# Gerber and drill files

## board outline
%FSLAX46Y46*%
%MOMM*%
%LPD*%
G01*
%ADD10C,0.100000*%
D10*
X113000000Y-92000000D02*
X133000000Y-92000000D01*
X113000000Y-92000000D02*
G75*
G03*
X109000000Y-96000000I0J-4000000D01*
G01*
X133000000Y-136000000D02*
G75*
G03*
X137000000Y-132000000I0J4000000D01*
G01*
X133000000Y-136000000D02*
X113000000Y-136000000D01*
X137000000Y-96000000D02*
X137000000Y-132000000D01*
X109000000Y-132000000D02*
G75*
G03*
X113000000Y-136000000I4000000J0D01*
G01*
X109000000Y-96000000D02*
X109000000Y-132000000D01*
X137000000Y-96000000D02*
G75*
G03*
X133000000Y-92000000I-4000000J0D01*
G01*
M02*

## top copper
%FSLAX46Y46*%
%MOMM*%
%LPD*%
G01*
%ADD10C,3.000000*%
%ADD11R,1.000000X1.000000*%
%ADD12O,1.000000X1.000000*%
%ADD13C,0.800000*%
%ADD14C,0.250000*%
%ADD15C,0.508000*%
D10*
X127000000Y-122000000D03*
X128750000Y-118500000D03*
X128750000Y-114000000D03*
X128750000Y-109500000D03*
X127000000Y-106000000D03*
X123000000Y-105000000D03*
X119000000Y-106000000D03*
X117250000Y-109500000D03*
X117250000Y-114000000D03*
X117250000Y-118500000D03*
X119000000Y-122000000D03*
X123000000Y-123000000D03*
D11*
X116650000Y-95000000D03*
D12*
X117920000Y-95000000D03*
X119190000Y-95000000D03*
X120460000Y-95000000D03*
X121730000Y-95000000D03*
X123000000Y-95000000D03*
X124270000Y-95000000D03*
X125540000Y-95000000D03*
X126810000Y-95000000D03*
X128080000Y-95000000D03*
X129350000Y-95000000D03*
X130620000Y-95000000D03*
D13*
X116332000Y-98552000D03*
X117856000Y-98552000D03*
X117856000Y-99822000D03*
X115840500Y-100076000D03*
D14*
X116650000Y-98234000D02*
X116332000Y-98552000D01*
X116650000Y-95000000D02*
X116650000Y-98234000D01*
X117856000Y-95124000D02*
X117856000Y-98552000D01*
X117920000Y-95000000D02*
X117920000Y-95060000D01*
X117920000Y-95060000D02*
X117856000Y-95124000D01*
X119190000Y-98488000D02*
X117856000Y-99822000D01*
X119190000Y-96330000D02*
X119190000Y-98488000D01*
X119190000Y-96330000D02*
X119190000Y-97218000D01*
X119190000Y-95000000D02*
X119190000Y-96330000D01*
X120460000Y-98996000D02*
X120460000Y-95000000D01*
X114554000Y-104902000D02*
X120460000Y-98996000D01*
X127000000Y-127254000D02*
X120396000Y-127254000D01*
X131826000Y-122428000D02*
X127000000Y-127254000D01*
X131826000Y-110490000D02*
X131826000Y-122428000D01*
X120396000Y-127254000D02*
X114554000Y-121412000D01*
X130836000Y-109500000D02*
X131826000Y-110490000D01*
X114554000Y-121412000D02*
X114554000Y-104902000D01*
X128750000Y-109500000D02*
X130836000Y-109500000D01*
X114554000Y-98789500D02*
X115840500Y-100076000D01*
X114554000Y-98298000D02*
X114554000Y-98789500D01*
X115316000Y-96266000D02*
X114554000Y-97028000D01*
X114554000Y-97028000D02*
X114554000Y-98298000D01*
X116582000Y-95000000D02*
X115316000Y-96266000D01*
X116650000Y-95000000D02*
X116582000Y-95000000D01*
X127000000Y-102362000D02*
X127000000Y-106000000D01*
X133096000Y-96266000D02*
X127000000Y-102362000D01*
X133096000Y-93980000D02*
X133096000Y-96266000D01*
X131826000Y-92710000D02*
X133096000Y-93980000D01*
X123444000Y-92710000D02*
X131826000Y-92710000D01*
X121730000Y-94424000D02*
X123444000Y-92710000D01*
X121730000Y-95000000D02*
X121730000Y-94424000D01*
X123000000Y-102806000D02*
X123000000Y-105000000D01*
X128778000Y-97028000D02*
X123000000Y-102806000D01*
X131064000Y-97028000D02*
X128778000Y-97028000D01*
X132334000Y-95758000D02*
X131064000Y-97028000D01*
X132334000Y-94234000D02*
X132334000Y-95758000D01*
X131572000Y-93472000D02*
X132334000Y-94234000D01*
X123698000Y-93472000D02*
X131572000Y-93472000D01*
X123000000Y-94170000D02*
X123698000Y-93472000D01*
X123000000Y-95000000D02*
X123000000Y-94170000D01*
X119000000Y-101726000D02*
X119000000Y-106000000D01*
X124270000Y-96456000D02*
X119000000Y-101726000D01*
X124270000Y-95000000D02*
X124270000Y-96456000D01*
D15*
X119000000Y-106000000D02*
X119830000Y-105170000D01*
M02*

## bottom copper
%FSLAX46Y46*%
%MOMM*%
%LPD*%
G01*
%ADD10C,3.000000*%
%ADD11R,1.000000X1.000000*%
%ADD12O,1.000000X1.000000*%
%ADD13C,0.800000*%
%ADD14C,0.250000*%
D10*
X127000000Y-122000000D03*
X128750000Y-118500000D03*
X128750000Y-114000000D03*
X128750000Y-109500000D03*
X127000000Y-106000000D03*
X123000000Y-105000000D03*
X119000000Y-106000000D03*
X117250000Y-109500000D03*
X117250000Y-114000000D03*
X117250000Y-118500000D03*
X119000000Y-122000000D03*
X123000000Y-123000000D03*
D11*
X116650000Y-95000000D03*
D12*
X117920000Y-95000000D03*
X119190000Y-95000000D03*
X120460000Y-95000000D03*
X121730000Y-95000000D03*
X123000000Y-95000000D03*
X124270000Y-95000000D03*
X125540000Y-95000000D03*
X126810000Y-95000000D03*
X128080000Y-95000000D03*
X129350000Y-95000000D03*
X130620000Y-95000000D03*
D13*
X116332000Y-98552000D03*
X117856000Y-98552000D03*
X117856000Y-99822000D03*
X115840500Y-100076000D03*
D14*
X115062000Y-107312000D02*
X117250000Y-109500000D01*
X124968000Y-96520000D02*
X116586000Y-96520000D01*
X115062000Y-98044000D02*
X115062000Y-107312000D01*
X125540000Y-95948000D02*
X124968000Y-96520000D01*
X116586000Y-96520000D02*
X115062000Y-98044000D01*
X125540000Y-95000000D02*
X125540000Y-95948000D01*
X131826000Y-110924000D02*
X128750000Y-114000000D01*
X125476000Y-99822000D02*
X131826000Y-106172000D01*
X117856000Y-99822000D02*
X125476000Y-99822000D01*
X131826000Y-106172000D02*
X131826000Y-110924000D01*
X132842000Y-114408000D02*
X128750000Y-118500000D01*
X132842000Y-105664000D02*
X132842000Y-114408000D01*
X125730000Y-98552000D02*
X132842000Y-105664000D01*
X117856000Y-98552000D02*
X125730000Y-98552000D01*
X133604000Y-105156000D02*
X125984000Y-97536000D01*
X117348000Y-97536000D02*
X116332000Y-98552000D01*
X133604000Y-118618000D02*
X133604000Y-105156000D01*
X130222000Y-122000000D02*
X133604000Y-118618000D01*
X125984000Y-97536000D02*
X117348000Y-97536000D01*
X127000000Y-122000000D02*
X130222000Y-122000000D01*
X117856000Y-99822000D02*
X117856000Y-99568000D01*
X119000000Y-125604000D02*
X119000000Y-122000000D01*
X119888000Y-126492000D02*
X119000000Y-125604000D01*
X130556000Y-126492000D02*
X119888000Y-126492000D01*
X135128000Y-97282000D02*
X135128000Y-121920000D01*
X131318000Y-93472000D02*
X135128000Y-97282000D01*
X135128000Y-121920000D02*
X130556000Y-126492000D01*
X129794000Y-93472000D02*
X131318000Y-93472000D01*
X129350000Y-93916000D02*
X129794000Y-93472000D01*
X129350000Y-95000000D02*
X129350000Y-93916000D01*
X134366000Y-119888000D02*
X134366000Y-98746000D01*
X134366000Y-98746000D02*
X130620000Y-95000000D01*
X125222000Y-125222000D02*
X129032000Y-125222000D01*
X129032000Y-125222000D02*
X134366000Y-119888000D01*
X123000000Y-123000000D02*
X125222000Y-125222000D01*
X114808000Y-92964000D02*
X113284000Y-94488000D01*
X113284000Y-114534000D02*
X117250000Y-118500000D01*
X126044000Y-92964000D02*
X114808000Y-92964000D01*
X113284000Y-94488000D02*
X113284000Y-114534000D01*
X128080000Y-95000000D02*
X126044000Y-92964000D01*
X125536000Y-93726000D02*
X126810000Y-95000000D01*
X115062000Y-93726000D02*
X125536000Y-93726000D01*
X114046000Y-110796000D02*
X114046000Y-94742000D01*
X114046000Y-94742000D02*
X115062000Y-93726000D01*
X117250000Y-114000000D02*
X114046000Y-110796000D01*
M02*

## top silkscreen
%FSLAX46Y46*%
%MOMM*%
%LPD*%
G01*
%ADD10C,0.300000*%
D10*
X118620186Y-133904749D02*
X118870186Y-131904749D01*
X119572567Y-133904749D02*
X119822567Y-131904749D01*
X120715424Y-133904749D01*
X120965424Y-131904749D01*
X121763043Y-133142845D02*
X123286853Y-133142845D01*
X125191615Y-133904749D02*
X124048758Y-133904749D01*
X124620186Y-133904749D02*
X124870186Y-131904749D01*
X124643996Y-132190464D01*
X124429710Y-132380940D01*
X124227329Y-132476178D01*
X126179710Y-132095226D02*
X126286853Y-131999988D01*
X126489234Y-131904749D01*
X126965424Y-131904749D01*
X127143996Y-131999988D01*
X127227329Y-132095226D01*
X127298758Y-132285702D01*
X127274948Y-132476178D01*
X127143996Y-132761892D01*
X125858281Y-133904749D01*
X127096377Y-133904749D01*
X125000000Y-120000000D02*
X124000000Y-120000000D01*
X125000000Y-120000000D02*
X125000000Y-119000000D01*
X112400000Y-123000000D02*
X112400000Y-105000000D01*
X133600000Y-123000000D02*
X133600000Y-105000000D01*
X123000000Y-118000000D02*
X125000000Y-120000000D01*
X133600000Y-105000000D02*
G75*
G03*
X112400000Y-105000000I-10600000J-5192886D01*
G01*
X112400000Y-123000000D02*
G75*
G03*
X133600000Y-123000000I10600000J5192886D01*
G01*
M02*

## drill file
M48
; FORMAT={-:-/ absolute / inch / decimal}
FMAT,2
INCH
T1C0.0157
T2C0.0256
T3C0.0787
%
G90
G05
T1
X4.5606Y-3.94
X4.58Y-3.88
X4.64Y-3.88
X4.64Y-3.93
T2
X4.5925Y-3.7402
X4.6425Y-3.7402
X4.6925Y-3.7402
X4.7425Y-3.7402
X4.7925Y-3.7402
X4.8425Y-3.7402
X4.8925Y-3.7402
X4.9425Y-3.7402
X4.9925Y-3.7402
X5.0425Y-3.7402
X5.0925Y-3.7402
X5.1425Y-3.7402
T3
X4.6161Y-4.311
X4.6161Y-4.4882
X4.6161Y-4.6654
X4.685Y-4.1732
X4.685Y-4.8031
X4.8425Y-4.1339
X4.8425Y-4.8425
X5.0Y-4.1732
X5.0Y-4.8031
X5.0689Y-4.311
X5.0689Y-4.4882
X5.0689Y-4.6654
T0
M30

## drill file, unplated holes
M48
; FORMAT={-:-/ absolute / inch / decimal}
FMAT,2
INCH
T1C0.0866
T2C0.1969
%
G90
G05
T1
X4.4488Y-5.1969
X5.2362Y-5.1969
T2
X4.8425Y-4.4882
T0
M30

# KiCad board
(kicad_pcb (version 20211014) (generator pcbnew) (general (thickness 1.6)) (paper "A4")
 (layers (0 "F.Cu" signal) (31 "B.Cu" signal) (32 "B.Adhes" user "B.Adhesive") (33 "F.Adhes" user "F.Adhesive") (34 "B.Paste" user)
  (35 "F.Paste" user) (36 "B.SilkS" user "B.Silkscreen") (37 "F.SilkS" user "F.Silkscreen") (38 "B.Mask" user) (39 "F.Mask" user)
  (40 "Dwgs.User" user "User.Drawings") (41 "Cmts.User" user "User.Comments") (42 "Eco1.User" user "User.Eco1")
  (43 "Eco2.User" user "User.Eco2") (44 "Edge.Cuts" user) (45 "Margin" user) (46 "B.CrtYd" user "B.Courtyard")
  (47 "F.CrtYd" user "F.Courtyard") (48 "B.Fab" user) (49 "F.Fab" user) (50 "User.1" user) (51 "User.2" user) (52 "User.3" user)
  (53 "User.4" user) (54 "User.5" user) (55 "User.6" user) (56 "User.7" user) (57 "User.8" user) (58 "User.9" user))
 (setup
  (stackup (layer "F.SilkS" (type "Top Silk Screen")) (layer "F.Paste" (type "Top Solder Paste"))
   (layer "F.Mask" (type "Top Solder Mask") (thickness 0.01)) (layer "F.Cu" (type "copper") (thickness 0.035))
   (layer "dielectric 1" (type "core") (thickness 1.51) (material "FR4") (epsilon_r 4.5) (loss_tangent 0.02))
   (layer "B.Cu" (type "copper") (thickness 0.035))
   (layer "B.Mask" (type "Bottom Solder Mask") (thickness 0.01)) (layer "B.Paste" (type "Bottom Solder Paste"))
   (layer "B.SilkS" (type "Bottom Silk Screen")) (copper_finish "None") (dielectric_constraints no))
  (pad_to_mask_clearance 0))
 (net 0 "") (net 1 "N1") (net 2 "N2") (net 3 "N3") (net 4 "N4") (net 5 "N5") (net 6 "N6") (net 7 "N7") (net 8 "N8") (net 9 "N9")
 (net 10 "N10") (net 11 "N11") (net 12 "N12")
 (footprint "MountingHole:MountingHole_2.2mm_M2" (layer "F.Cu") (at 113 132)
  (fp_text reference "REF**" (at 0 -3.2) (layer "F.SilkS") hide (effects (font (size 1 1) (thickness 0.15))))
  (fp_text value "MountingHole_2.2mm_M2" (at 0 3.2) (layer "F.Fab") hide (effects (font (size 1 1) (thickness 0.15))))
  (pad "" np_thru_hole circle (at 0 0) (size 2.2 2.2) (drill 2.2) (layers *.Cu *.Mask)))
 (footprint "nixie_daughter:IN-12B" (layer "F.Cu") (at 123 114)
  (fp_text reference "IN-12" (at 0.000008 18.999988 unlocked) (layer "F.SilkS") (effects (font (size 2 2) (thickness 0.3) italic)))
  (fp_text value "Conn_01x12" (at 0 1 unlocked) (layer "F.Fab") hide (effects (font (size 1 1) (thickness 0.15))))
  (fp_line (start 2 6) (end 2 5) (layer "F.SilkS") (width 0.3))
  (fp_line (start 2 6) (end 1 6) (layer "F.SilkS") (width 0.3))
  (fp_line (start 0 4) (end 2 6) (layer "F.SilkS") (width 0.3))
  (fp_line (start -10.6 9) (end -10.6 -9) (layer "F.SilkS") (width 0.3))
  (fp_line (start 10.6 9) (end 10.6 -9) (layer "F.SilkS") (width 0.3))
  (fp_arc (start -10.6 -9) (mid 0 -15.61076) (end 10.6 -9) (layer "F.SilkS") (width 0.3))
  (fp_arc (start 10.6 9) (mid 0 15.61076) (end -10.6 9) (layer "F.SilkS") (width 0.3))
  (pad "" np_thru_hole circle (at 0 0 180) (size 5 5) (drill 5) (layers *.Mask))
  (pad "1" thru_hole circle (at 4 8 180) (size 3 3) (drill 2) (layers *.Cu *.Mask) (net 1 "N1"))
  (pad "2" thru_hole circle (at 5.75 4.5) (size 3 3) (drill 2) (layers *.Cu *.Mask) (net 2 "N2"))
  (pad "3" thru_hole circle (at 5.75 0) (size 3 3) (drill 2) (layers *.Cu *.Mask) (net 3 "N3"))
  (pad "4" thru_hole circle (at 5.75 -4.5) (size 3 3) (drill 2) (layers *.Cu *.Mask) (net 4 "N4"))
  (pad "5" thru_hole circle (at 4 -8) (size 3 3) (drill 2) (layers *.Cu *.Mask) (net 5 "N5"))
  (pad "6" thru_hole circle (at 0 -9) (size 3 3) (drill 2) (layers *.Cu *.Mask) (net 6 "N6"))
  (pad "7" thru_hole circle (at -4 -8) (size 3 3) (drill 2) (layers *.Cu *.Mask) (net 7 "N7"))
  (pad "8" thru_hole circle (at -5.75 -4.5) (size 3 3) (drill 2) (layers *.Cu *.Mask) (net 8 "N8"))
  (pad "9" thru_hole circle (at -5.75 0) (size 3 3) (drill 2) (layers *.Cu *.Mask) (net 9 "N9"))
  (pad "10" thru_hole circle (at -5.75 4.5) (size 3 3) (drill 2) (layers *.Cu *.Mask) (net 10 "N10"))
  (pad "11" thru_hole circle (at -4 8 180) (size 3 3) (drill 2) (layers *.Cu *.Mask) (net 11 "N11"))
  (pad "12" thru_hole circle (at 0 9) (size 3 3) (drill 2) (layers *.Cu *.Mask) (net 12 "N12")))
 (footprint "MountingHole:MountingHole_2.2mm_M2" (layer "F.Cu") (at 133 132)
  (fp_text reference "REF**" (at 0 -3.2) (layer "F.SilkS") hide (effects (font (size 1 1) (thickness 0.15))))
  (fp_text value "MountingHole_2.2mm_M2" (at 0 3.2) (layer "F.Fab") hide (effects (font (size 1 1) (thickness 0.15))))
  (pad "" np_thru_hole circle (at 0 0) (size 2.2 2.2) (drill 2.2) (layers *.Cu *.Mask)))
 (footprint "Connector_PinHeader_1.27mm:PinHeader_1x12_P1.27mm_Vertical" (layer "B.Cu") (at 116.65 95 -90)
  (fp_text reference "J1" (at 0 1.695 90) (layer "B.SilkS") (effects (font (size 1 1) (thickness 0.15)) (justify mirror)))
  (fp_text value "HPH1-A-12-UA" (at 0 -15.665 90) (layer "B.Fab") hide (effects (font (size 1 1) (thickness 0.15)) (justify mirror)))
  (pad "1" thru_hole rect (at 0 0 270) (size 1 1) (drill 0.65) (layers *.Cu *.Mask) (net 1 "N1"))
  (pad "2" thru_hole oval (at 0 -1.27 270) (size 1 1) (drill 0.65) (layers *.Cu *.Mask) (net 2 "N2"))
  (pad "3" thru_hole oval (at 0 -2.54 270) (size 1 1) (drill 0.65) (layers *.Cu *.Mask) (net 3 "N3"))
  (pad "4" thru_hole oval (at 0 -3.81 270) (size 1 1) (drill 0.65) (layers *.Cu *.Mask) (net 4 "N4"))
  (pad "5" thru_hole oval (at 0 -5.08 270) (size 1 1) (drill 0.65) (layers *.Cu *.Mask) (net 5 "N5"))
  (pad "6" thru_hole oval (at 0 -6.35 270) (size 1 1) (drill 0.65) (layers *.Cu *.Mask) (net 6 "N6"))
  (pad "7" thru_hole oval (at 0 -7.62 270) (size 1 1) (drill 0.65) (layers *.Cu *.Mask) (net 7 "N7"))
  (pad "8" thru_hole oval (at 0 -8.89 270) (size 1 1) (drill 0.65) (layers *.Cu *.Mask) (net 8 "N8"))
  (pad "9" thru_hole oval (at 0 -10.16 270) (size 1 1) (drill 0.65) (layers *.Cu *.Mask) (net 9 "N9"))
  (pad "10" thru_hole oval (at 0 -11.43 270) (size 1 1) (drill 0.65) (layers *.Cu *.Mask) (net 10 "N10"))
  (pad "11" thru_hole oval (at 0 -12.7 270) (size 1 1) (drill 0.65) (layers *.Cu *.Mask) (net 11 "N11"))
  (pad "12" thru_hole oval (at 0 -13.97 270) (size 1 1) (drill 0.65) (layers *.Cu *.Mask) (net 12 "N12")))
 (gr_line (start 113 92) (end 133 92) (layer "Edge.Cuts") (width 0.1))
 (gr_arc (start 109 96) (mid 110.171573 93.171573) (end 113 92) (layer "Edge.Cuts") (width 0.1))
 (gr_arc (start 137 132) (mid 135.828427 134.828427) (end 133 136) (layer "Edge.Cuts") (width 0.1))
 (gr_line (start 133 136) (end 113 136) (layer "Edge.Cuts") (width 0.1))
 (gr_line (start 137 96) (end 137 132) (layer "Edge.Cuts") (width 0.1))
 (gr_arc (start 113 136) (mid 110.171573 134.828427) (end 109 132) (layer "Edge.Cuts") (width 0.1))
 (gr_line (start 109 96) (end 109 132) (layer "Edge.Cuts") (width 0.1))
 (gr_arc (start 133 92) (mid 135.828427 93.171573) (end 137 96) (layer "Edge.Cuts") (width 0.1))
 (segment (start 116.65 95) (end 116.582 95) (width 0.25) (layer "F.Cu") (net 1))
 (segment (start 115.316 96.266) (end 114.554 97.028) (width 0.25) (layer "F.Cu") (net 1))
 (segment (start 114.554 98.298) (end 114.554 98.7895) (width 0.25) (layer "F.Cu") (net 1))
 (segment (start 116.65 95) (end 116.65 98.234) (width 0.25) (layer "F.Cu") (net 1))
 (segment (start 114.554 98.7895) (end 115.8405 100.076) (width 0.25) (layer "F.Cu") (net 1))
 (segment (start 116.65 98.234) (end 116.332 98.552) (width 0.25) (layer "F.Cu") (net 1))
 (segment (start 116.582 95) (end 115.316 96.266) (width 0.25) (layer "F.Cu") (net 1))
 (segment (start 114.554 97.028) (end 114.554 98.298) (width 0.25) (layer "F.Cu") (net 1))
 (via (at 115.8405 100.076) (size 0.8) (drill 0.4) (layers "F.Cu" "B.Cu") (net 1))
 (via (at 116.332 98.552) (size 0.8) (drill 0.4) (layers "F.Cu" "B.Cu") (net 1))
 (segment (start 130.222 122) (end 133.604 118.618) (width 0.25) (layer "B.Cu") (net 1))
 (segment (start 133.604 118.618) (end 133.604 105.156) (width 0.25) (layer "B.Cu") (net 1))
 (segment (start 133.604 105.156) (end 125.984 97.536) (width 0.25) (layer "B.Cu") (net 1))
 (segment (start 117.348 97.536) (end 116.332 98.552) (width 0.25) (layer "B.Cu") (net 1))
 (segment (start 127 122) (end 130.222 122) (width 0.25) (layer "B.Cu") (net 1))
 (segment (start 125.984 97.536) (end 117.348 97.536) (width 0.25) (layer "B.Cu") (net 1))
 (segment (start 117.92 95) (end 117.92 95.06) (width 0.25) (layer "F.Cu") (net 2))
 (segment (start 117.856 95.124) (end 117.856 98.552) (width 0.25) (layer "F.Cu") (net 2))
 (segment (start 117.92 95.06) (end 117.856 95.124) (width 0.25) (layer "F.Cu") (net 2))
 (via (at 117.856 98.552) (size 0.8) (drill 0.4) (layers "F.Cu" "B.Cu") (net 2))
 (segment (start 132.842 105.664) (end 132.842 114.408) (width 0.25) (layer "B.Cu") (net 2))
 (segment (start 117.856 98.552) (end 125.73 98.552) (width 0.25) (layer "B.Cu") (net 2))
 (segment (start 132.842 114.408) (end 128.75 118.5) (width 0.25) (layer "B.Cu") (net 2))
 (segment (start 125.73 98.552) (end 132.842 105.664) (width 0.25) (layer "B.Cu") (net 2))
 (segment (start 119.19 96.33) (end 119.19 97.218) (width 0.25) (layer "F.Cu") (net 3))
 (segment (start 119.19 96.33) (end 119.19 98.488) (width 0.25) (layer "F.Cu") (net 3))
 (segment (start 119.19 95) (end 119.19 96.33) (width 0.25) (layer "F.Cu") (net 3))
 (segment (start 119.19 98.488) (end 117.856 99.822) (width 0.25) (layer "F.Cu") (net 3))
 (via (at 117.856 99.822) (size 0.8) (drill 0.4) (layers "F.Cu" "B.Cu") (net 3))
 (segment (start 131.826 106.172) (end 131.826 110.924) (width 0.25) (layer "B.Cu") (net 3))
 (segment (start 131.826 110.924) (end 128.75 114) (width 0.25) (layer "B.Cu") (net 3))
 (segment (start 125.476 99.822) (end 131.826 106.172) (width 0.25) (layer "B.Cu") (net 3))
 (segment (start 117.856 99.822) (end 117.856 99.568) (width 0.25) (layer "B.Cu") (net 3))
 (segment (start 117.856 99.822) (end 125.476 99.822) (width 0.25) (layer "B.Cu") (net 3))
 (segment (start 114.554 121.412) (end 114.554 104.902) (width 0.25) (layer "F.Cu") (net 4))
 (segment (start 128.75 109.5) (end 130.836 109.5) (width 0.25) (layer "F.Cu") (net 4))
 (segment (start 130.836 109.5) (end 131.826 110.49) (width 0.25) (layer "F.Cu") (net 4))
 (segment (start 114.554 104.902) (end 120.46 98.996) (width 0.25) (layer "F.Cu") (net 4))
 (segment (start 131.826 110.49) (end 131.826 122.428) (width 0.25) (layer "F.Cu") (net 4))
 (segment (start 131.826 122.428) (end 127 127.254) (width 0.25) (layer "F.Cu") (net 4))
 (segment (start 120.46 98.996) (end 120.46 95) (width 0.25) (layer "F.Cu") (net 4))
 (segment (start 120.396 127.254) (end 114.554 121.412) (width 0.25) (layer "F.Cu") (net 4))
 (segment (start 127 127.254) (end 120.396 127.254) (width 0.25) (layer "F.Cu") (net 4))
 (segment (start 133.096 93.98) (end 133.096 96.266) (width 0.25) (layer "F.Cu") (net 5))
 (segment (start 133.096 96.266) (end 127 102.362) (width 0.25) (layer "F.Cu") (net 5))
 (segment (start 121.73 95) (end 121.73 94.424) (width 0.25) (layer "F.Cu") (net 5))
 (segment (start 123.444 92.71) (end 131.826 92.71) (width 0.25) (layer "F.Cu") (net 5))
 (segment (start 131.826 92.71) (end 133.096 93.98) (width 0.25) (layer "F.Cu") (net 5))
 (segment (start 121.73 94.424) (end 123.444 92.71) (width 0.25) (layer "F.Cu") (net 5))
 (segment (start 127 102.362) (end 127 106) (width 0.25) (layer "F.Cu") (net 5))
 (segment (start 131.572 93.472) (end 132.334 94.234) (width 0.25) (layer "F.Cu") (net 6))
 (segment (start 123 102.806) (end 123 105) (width 0.25) (layer "F.Cu") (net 6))
 (segment (start 128.778 97.028) (end 123 102.806) (width 0.25) (layer "F.Cu") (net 6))
 (segment (start 132.334 95.758) (end 131.064 97.028) (width 0.25) (layer "F.Cu") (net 6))
 (segment (start 123 95) (end 123 94.17) (width 0.25) (layer "F.Cu") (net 6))
 (segment (start 131.064 97.028) (end 128.778 97.028) (width 0.25) (layer "F.Cu") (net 6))
 (segment (start 123.698 93.472) (end 131.572 93.472) (width 0.25) (layer "F.Cu") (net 6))
 (segment (start 132.334 94.234) (end 132.334 95.758) (width 0.25) (layer "F.Cu") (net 6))
 (segment (start 123 94.17) (end 123.698 93.472) (width 0.25) (layer "F.Cu") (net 6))
 (segment (start 119 106) (end 119.83 105.17) (width 0.508) (layer "F.Cu") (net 7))
 (segment (start 119 101.726) (end 119 106) (width 0.25) (layer "F.Cu") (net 7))
 (segment (start 124.27 95) (end 124.27 96.456) (width 0.25) (layer "F.Cu") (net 7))
 (segment (start 124.27 96.456) (end 119 101.726) (width 0.25) (layer "F.Cu") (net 7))
 (segment (start 124.968 96.52) (end 116.586 96.52) (width 0.25) (layer "B.Cu") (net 8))
 (segment (start 116.586 96.52) (end 115.062 98.044) (width 0.25) (layer "B.Cu") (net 8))
 (segment (start 115.062 98.044) (end 115.062 107.312) (width 0.25) (layer "B.Cu") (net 8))
 (segment (start 115.062 107.312) (end 117.25 109.5) (width 0.25) (layer "B.Cu") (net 8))
 (segment (start 125.54 95.948) (end 124.968 96.52) (width 0.25) (layer "B.Cu") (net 8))
 (segment (start 125.54 95) (end 125.54 95.948) (width 0.25) (layer "B.Cu") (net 8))
 (segment (start 117.25 114) (end 114.046 110.796) (width 0.25) (layer "B.Cu") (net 9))
 (segment (start 115.062 93.726) (end 125.536 93.726) (width 0.25) (layer "B.Cu") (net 9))
 (segment (start 114.046 110.796) (end 114.046 94.742) (width 0.25) (layer "B.Cu") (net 9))
 (segment (start 114.046 94.742) (end 115.062 93.726) (width 0.25) (layer "B.Cu") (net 9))
 (segment (start 125.536 93.726) (end 126.81 95) (width 0.25) (layer "B.Cu") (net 9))
 (segment (start 113.284 94.488) (end 113.284 114.534) (width 0.25) (layer "B.Cu") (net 10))
 (segment (start 126.044 92.964) (end 114.808 92.964) (width 0.25) (layer "B.Cu") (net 10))
 (segment (start 113.284 114.534) (end 117.25 118.5) (width 0.25) (layer "B.Cu") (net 10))
 (segment (start 128.08 95) (end 126.044 92.964) (width 0.25) (layer "B.Cu") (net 10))
 (segment (start 114.808 92.964) (end 113.284 94.488) (width 0.25) (layer "B.Cu") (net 10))
 (segment (start 129.794 93.472) (end 131.318 93.472) (width 0.25) (layer "B.Cu") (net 11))
 (segment (start 130.556 126.492) (end 119.888 126.492) (width 0.25) (layer "B.Cu") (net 11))
 (segment (start 129.35 95) (end 129.35 93.916) (width 0.25) (layer "B.Cu") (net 11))
 (segment (start 131.318 93.472) (end 135.128 97.282) (width 0.25) (layer "B.Cu") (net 11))
 (segment (start 119.888 126.492) (end 119 125.604) (width 0.25) (layer "B.Cu") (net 11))
 (segment (start 129.35 93.916) (end 129.794 93.472) (width 0.25) (layer "B.Cu") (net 11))
 (segment (start 119 125.604) (end 119 122) (width 0.25) (layer "B.Cu") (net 11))
 (segment (start 135.128 121.92) (end 130.556 126.492) (width 0.25) (layer "B.Cu") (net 11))
 (segment (start 135.128 97.282) (end 135.128 121.92) (width 0.25) (layer "B.Cu") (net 11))
 (segment (start 125.222 125.222) (end 129.032 125.222) (width 0.25) (layer "B.Cu") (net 12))
 (segment (start 123 123) (end 125.222 125.222) (width 0.25) (layer "B.Cu") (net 12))
 (segment (start 129.032 125.222) (end 134.366 119.888) (width 0.25) (layer "B.Cu") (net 12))
 (segment (start 134.366 98.746) (end 130.62 95) (width 0.25) (layer "B.Cu") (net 12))
 (segment (start 134.366 119.888) (end 134.366 98.746) (width 0.25) (layer "B.Cu") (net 12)))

